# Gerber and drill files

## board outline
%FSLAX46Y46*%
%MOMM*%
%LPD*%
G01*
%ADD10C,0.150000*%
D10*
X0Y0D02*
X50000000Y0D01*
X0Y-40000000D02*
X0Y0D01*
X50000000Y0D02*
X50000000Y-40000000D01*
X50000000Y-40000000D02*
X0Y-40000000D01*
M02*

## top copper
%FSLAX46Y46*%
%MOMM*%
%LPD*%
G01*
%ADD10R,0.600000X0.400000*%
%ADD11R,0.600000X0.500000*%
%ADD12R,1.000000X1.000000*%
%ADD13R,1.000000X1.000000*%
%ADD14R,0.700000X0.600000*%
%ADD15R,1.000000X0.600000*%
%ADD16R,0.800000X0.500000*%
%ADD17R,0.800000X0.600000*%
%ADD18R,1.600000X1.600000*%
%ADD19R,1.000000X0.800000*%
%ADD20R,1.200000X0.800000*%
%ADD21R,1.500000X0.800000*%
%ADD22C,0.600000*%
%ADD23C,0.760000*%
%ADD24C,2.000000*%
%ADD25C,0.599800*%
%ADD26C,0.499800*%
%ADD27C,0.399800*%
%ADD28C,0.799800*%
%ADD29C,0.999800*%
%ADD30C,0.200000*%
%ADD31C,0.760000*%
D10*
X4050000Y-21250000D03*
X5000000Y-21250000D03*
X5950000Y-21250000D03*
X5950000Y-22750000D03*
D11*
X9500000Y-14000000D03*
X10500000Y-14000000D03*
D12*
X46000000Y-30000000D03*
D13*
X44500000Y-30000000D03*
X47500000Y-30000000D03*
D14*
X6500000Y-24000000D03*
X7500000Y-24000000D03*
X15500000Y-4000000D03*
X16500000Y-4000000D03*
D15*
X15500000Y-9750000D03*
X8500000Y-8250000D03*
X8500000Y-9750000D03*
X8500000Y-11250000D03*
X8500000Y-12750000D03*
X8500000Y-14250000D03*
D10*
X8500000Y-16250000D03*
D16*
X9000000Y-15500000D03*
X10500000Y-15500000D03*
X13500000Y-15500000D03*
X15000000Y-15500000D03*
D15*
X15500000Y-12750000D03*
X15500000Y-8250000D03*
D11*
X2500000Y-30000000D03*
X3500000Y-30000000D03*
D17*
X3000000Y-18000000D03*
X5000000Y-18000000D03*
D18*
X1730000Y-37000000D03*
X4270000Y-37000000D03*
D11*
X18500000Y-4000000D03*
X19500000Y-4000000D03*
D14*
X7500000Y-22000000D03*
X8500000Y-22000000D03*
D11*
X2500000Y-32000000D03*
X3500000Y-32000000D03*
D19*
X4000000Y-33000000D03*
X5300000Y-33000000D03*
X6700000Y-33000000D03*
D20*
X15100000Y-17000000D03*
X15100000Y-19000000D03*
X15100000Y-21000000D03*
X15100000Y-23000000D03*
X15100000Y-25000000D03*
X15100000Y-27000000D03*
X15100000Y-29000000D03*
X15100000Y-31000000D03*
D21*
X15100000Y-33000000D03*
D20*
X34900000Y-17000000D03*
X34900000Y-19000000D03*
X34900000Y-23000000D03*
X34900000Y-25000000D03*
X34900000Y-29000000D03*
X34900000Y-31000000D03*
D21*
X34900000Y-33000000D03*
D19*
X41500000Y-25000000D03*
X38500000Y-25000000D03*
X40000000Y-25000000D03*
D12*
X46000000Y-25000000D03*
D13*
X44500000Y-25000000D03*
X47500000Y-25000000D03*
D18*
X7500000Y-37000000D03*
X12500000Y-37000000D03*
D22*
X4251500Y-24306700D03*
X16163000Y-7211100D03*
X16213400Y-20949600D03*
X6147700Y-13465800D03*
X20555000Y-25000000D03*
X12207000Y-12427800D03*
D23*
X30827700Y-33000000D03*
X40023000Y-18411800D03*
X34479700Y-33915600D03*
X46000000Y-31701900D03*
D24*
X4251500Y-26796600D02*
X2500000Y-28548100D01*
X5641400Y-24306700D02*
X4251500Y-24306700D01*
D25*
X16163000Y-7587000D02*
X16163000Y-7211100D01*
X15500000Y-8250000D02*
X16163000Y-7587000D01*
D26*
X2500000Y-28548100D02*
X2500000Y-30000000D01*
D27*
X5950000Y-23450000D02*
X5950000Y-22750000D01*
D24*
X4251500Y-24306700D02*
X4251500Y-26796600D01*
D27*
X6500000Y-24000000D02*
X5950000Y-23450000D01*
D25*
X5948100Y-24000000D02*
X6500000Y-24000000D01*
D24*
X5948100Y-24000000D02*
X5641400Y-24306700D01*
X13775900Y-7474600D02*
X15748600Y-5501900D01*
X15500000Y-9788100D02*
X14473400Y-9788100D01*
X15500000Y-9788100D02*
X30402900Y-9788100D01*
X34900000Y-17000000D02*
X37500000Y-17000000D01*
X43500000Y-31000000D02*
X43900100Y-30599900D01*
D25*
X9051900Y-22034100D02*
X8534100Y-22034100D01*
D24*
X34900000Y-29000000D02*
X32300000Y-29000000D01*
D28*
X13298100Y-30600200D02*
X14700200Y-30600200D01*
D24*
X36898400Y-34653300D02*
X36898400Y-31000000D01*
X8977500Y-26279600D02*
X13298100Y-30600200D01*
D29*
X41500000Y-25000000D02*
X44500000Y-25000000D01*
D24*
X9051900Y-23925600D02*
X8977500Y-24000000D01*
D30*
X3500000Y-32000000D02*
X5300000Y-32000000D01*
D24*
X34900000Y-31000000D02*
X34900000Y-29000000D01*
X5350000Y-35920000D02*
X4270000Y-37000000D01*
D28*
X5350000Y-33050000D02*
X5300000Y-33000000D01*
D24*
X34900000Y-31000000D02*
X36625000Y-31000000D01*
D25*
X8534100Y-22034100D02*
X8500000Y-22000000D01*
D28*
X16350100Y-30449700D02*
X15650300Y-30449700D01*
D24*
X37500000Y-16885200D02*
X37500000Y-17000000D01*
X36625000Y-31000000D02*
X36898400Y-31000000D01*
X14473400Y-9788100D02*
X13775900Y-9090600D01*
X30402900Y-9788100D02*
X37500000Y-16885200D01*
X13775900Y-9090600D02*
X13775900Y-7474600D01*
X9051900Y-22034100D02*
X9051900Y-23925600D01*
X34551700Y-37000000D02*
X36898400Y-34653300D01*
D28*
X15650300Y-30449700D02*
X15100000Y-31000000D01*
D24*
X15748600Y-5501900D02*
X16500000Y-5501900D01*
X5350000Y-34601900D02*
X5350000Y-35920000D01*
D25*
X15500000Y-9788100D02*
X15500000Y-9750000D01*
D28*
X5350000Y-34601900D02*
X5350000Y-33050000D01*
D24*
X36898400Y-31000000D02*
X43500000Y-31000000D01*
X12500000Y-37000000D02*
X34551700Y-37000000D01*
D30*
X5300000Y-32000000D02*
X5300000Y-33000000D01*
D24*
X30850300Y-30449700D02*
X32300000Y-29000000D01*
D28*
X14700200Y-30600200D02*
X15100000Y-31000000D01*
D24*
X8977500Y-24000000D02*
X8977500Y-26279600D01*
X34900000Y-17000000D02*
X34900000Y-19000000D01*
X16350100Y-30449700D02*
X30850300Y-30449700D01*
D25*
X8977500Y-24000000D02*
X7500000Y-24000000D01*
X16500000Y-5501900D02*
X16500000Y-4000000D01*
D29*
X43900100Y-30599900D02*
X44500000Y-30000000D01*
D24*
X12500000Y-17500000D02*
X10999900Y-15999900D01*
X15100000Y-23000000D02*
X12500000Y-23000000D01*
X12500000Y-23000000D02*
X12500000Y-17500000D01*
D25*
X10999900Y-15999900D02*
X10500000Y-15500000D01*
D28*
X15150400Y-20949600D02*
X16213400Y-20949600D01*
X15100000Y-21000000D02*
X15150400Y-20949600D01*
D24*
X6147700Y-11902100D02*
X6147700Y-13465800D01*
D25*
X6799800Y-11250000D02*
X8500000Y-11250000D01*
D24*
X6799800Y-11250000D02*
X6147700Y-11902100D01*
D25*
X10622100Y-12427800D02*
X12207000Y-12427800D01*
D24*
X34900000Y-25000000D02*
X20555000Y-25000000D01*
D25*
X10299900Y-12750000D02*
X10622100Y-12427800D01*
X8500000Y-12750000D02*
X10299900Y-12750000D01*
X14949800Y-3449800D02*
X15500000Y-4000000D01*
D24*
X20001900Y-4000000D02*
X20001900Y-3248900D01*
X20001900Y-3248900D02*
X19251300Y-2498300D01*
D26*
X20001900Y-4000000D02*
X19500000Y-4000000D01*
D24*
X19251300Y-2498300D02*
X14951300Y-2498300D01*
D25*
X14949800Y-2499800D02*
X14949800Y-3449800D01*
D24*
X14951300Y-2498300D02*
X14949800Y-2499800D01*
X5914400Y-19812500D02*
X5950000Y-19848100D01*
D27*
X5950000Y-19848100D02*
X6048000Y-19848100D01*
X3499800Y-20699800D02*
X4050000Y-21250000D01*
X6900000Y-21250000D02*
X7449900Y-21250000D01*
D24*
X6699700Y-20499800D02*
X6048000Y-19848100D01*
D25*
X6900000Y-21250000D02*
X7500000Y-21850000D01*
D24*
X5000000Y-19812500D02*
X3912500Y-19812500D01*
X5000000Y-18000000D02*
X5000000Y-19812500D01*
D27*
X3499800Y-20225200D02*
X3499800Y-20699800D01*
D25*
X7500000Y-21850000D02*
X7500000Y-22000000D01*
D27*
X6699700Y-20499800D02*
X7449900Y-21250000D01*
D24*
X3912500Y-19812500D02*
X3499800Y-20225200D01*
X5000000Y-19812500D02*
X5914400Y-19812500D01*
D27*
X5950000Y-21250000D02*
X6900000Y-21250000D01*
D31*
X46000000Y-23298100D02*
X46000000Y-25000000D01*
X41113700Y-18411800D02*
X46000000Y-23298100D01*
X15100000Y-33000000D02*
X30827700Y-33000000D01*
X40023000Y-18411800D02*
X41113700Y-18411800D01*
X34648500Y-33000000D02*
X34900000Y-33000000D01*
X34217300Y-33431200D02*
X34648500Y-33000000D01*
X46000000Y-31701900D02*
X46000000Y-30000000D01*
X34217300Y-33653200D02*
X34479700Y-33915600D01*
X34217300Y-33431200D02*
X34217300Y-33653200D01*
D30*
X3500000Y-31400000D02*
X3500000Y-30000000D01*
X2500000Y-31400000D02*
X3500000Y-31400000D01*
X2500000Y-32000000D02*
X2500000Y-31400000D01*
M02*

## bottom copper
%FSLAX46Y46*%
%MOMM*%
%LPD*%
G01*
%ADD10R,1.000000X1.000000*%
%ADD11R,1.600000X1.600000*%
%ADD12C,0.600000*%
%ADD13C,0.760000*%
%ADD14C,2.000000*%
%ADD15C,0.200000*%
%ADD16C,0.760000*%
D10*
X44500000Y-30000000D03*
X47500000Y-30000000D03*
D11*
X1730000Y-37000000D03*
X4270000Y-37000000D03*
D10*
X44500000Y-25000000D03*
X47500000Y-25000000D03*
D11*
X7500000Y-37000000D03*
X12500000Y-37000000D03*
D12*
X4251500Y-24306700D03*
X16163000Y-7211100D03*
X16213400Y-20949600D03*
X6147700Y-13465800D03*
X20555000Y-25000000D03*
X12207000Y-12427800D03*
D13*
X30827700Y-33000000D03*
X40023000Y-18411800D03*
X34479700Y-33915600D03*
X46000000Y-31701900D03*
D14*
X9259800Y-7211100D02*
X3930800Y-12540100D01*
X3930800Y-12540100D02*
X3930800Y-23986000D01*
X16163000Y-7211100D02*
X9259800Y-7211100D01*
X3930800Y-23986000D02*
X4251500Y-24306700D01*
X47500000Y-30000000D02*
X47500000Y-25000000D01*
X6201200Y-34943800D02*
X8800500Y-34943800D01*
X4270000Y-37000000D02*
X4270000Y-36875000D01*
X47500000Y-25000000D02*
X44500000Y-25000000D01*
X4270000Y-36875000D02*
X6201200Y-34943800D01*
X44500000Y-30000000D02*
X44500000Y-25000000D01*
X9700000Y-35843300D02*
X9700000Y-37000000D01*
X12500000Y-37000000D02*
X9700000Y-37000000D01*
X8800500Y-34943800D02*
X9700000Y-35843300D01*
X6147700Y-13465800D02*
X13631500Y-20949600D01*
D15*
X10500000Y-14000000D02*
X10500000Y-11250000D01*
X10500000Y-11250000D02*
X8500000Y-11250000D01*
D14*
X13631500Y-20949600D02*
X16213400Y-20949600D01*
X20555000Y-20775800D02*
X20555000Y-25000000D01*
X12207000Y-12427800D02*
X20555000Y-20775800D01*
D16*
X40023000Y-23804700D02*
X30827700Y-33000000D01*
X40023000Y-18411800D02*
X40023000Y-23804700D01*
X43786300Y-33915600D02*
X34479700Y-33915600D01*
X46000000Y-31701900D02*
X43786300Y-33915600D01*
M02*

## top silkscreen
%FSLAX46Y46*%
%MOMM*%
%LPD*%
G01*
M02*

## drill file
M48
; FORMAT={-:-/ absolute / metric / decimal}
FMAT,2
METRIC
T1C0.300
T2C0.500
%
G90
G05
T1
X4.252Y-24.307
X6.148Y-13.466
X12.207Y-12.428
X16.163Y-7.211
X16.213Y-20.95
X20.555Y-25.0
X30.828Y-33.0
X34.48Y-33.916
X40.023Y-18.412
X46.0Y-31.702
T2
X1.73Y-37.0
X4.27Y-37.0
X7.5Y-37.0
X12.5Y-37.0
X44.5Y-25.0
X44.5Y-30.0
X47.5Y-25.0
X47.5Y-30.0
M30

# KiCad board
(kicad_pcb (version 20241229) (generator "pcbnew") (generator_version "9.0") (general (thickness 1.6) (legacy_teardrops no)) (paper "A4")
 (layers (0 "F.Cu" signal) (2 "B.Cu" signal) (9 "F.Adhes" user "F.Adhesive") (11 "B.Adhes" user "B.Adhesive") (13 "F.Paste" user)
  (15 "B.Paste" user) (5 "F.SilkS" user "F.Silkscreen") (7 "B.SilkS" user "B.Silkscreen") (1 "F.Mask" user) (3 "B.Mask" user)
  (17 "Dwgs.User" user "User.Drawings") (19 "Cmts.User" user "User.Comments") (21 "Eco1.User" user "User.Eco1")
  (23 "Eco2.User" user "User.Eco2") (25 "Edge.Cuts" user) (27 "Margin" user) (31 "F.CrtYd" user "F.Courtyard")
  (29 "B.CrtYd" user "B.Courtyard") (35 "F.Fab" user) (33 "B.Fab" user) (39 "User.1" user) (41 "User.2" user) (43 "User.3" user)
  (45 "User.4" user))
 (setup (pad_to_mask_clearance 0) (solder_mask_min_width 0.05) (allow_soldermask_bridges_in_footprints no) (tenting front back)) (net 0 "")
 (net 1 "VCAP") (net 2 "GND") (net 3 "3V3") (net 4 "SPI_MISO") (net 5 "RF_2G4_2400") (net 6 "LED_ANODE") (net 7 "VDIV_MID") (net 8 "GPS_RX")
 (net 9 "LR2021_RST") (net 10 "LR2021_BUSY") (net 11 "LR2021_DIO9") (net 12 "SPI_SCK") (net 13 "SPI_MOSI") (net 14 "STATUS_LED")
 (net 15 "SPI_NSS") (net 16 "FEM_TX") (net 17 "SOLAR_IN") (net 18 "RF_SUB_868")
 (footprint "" (layer "F.Cu") (at 5 22)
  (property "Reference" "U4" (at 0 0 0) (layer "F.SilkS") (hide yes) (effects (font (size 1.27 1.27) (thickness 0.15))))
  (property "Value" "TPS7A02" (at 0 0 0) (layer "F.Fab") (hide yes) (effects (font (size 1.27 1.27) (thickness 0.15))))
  (pad "1" smd rect (at -0.95 -0.75) (size 0.6 0.4) (layers "F.Cu" "F.Mask") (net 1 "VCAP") (thermal_bridge_angle 45))
  (pad "2" smd rect (at 0 -0.75) (size 0.6 0.4) (layers "F.Cu" "F.Mask") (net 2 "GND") (thermal_bridge_angle 45))
  (pad "3" smd rect (at 0.95 -0.75) (size 0.6 0.4) (layers "F.Cu" "F.Mask") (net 1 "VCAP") (thermal_bridge_angle 45))
  (pad "4" smd rect (at 0.95 0.75) (size 0.6 0.4) (layers "F.Cu" "F.Mask") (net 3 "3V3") (thermal_bridge_angle 45)))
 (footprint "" (layer "F.Cu") (at 10 14)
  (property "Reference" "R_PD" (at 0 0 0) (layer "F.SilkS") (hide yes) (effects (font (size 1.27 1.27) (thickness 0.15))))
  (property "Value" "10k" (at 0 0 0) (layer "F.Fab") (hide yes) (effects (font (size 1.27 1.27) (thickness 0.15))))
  (pad "1" smd rect (at -0.5 0) (size 0.6 0.5) (layers "F.Cu" "F.Mask") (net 2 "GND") (thermal_bridge_angle 45))
  (pad "2" smd rect (at 0.5 0) (size 0.6 0.5) (layers "F.Cu" "F.Mask") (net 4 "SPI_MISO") (thermal_bridge_angle 45)))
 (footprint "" (layer "F.Cu") (at 46 30)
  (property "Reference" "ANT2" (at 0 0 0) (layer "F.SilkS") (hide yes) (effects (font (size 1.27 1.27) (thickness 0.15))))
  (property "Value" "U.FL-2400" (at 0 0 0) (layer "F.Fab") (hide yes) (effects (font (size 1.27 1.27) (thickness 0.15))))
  (pad "1" smd rect (at 0 0) (size 1 1) (layers "F.Cu" "F.Mask") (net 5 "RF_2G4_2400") (thermal_bridge_angle 45))
  (pad "2" thru_hole rect (at -1.5 0) (size 1 1) (drill 0.5) (layers "*.Cu" "*.Mask") (remove_unused_layers no) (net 2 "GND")
   (thermal_bridge_angle 45))
  (pad "3" thru_hole rect (at 1.5 0) (size 1 1) (drill 0.5) (layers "*.Cu" "*.Mask") (remove_unused_layers no) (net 2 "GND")
   (thermal_bridge_angle 45)))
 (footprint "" (layer "F.Cu") (at 7 24)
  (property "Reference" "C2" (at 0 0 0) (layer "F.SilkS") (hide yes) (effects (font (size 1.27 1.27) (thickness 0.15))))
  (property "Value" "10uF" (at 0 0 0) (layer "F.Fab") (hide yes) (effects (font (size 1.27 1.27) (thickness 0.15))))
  (pad "1" smd rect (at -0.5 0) (size 0.7 0.6) (layers "F.Cu" "F.Mask") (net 3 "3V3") (thermal_bridge_angle 45))
  (pad "2" smd rect (at 0.5 0) (size 0.7 0.6) (layers "F.Cu" "F.Mask") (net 2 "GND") (thermal_bridge_angle 45)))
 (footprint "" (layer "F.Cu") (at 16 4)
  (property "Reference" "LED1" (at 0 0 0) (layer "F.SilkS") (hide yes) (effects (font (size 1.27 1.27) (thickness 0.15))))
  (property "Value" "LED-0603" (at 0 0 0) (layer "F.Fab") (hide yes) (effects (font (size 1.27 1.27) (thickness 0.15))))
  (pad "A" smd rect (at -0.5 0) (size 0.7 0.6) (layers "F.Cu" "F.Mask") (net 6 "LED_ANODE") (thermal_bridge_angle 45))
  (pad "K" smd rect (at 0.5 0) (size 0.7 0.6) (layers "F.Cu" "F.Mask") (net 2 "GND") (thermal_bridge_angle 45)))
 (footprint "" (layer "F.Cu") (at 12 12)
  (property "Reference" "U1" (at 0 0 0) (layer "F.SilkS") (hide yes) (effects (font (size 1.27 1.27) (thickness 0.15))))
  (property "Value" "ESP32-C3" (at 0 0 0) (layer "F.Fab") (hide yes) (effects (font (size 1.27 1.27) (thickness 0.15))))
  (pad "GND" smd rect (at 3.5 -2.25) (size 1 0.6) (layers "F.Cu" "F.Mask") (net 2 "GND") (thermal_bridge_angle 45))
  (pad "GPIO0" smd rect (at -3.5 -3.75) (size 1 0.6) (layers "F.Cu" "F.Mask") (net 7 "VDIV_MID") (thermal_bridge_angle 45))
  (pad "GPIO1" smd rect (at -3.5 -2.25) (size 1 0.6) (layers "F.Cu" "F.Mask") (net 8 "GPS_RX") (thermal_bridge_angle 45))
  (pad "GPIO2" smd rect (at -3.5 -0.75) (size 1 0.6) (layers "F.Cu" "F.Mask") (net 4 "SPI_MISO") (thermal_bridge_angle 45))
  (pad "GPIO3" smd rect (at -3.5 0.75) (size 1 0.6) (layers "F.Cu" "F.Mask") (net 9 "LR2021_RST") (thermal_bridge_angle 45))
  (pad "GPIO4" smd rect (at -3.5 2.25) (size 1 0.6) (layers "F.Cu" "F.Mask") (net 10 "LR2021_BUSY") (thermal_bridge_angle 45))
  (pad "GPIO5" smd rect (at -3.5 4.25) (size 0.6 0.4) (layers "F.Cu" "F.Mask") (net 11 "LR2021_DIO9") (thermal_bridge_angle 45))
  (pad "GPIO6" smd rect (at -3 3.5) (size 0.8 0.5) (layers "F.Cu" "F.Mask") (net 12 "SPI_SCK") (thermal_bridge_angle 45))
  (pad "GPIO7" smd rect (at -1.5 3.5) (size 0.8 0.5) (layers "F.Cu" "F.Mask") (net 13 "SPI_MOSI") (thermal_bridge_angle 45))
  (pad "GPIO9" smd rect (at 1.5 3.5) (size 0.8 0.5) (layers "F.Cu" "F.Mask") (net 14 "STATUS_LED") (thermal_bridge_angle 45))
  (pad "GPIO10" smd rect (at 3 3.5) (size 0.8 0.5) (layers "F.Cu" "F.Mask") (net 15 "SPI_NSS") (thermal_bridge_angle 45))
  (pad "GPIO19" smd rect (at 3.5 0.75) (size 1 0.6) (layers "F.Cu" "F.Mask") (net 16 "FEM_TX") (thermal_bridge_angle 45))
  (pad "VCC" smd rect (at 3.5 -3.75) (size 1 0.6) (layers "F.Cu" "F.Mask") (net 3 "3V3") (thermal_bridge_angle 45)))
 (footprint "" (layer "F.Cu") (at 3 30)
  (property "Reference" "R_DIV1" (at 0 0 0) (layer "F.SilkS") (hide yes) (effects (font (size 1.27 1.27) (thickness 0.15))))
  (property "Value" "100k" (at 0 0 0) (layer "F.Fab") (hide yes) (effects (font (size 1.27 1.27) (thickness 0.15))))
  (pad "1" smd rect (at -0.5 0) (size 0.6 0.5) (layers "F.Cu" "F.Mask") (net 3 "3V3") (thermal_bridge_angle 45))
  (pad "2" smd rect (at 0.5 0) (size 0.6 0.5) (layers "F.Cu" "F.Mask") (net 7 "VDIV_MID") (thermal_bridge_angle 45)))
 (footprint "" (layer "F.Cu") (at 4 18)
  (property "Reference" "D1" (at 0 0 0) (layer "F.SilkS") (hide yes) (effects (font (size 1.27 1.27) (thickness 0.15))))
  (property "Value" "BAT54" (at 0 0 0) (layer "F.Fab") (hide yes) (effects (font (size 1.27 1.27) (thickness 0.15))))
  (pad "A" smd rect (at -1 0) (size 0.8 0.6) (layers "F.Cu" "F.Mask") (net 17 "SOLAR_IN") (thermal_bridge_angle 45))
  (pad "K" smd rect (at 1 0) (size 0.8 0.6) (layers "F.Cu" "F.Mask") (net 1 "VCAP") (thermal_bridge_angle 45)))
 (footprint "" (layer "F.Cu") (at 3 37)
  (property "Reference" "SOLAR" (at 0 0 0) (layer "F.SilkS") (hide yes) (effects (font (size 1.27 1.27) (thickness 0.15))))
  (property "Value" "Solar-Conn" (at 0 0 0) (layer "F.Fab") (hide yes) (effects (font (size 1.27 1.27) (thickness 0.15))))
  (pad "1" thru_hole rect (at -1.27 0) (size 1.6 1.6) (drill 0.5) (layers "*.Cu" "*.Mask") (remove_unused_layers no) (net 17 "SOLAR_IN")
   (thermal_bridge_angle 45))
  (pad "2" thru_hole rect (at 1.27 0) (size 1.6 1.6) (drill 0.5) (layers "*.Cu" "*.Mask") (remove_unused_layers no) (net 2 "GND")
   (thermal_bridge_angle 45)))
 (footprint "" (layer "F.Cu") (at 19 4)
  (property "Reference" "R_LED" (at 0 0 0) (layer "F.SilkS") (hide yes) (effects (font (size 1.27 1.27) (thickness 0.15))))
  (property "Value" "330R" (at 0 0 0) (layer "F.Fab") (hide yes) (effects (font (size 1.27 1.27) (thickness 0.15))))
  (pad "1" smd rect (at -0.5 0) (size 0.6 0.5) (layers "F.Cu" "F.Mask") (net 14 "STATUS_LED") (thermal_bridge_angle 45))
  (pad "2" smd rect (at 0.5 0) (size 0.6 0.5) (layers "F.Cu" "F.Mask") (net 6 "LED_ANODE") (thermal_bridge_angle 45)))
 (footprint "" (layer "F.Cu") (at 8 22)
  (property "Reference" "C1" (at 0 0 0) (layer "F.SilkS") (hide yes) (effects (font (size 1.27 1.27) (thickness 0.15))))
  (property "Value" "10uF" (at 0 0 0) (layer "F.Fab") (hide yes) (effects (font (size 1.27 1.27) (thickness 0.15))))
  (pad "1" smd rect (at -0.5 0) (size 0.7 0.6) (layers "F.Cu" "F.Mask") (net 1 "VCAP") (thermal_bridge_angle 45))
  (pad "2" smd rect (at 0.5 0) (size 0.7 0.6) (layers "F.Cu" "F.Mask") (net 2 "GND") (thermal_bridge_angle 45)))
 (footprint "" (layer "F.Cu") (at 3 32)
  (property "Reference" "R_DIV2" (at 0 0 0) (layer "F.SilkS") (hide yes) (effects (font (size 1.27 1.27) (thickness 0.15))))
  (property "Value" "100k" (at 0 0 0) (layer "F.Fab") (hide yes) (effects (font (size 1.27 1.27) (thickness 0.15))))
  (pad "1" smd rect (at -0.5 0) (size 0.6 0.5) (layers "F.Cu" "F.Mask") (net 7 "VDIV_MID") (thermal_bridge_angle 45))
  (pad "2" smd rect (at 0.5 0) (size 0.6 0.5) (layers "F.Cu" "F.Mask") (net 2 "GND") (thermal_bridge_angle 45)))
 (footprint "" (layer "F.Cu") (at 6 33)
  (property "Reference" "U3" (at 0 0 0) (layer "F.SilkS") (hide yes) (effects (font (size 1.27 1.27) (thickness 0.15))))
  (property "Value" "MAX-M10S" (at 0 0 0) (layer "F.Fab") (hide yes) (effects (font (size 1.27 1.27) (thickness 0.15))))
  (pad "1" smd rect (at -2 0) (size 1 0.8) (layers "F.Cu" "F.Mask") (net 3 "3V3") (thermal_bridge_angle 45))
  (pad "2" smd rect (at -0.7 0) (size 1 0.8) (layers "F.Cu" "F.Mask") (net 2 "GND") (thermal_bridge_angle 45))
  (pad "3" smd rect (at 0.7 0) (size 1 0.8) (layers "F.Cu" "F.Mask") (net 8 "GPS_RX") (thermal_bridge_angle 45)))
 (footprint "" (layer "F.Cu") (at 25 25)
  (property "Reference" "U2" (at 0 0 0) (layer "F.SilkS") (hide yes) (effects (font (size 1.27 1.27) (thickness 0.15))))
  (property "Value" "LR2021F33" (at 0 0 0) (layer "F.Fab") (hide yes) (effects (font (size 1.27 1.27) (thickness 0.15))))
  (pad "1" smd rect (at -9.9 -8) (size 1.2 0.8) (layers "F.Cu" "F.Mask") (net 3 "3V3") (thermal_bridge_angle 45))
  (pad "2" smd rect (at -9.9 -6) (size 1.2 0.8) (layers "F.Cu" "F.Mask") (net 2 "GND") (thermal_bridge_angle 45))
  (pad "3" smd rect (at -9.9 -4) (size 1.2 0.8) (layers "F.Cu" "F.Mask") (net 4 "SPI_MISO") (thermal_bridge_angle 45))
  (pad "4" smd rect (at -9.9 -2) (size 1.2 0.8) (layers "F.Cu" "F.Mask") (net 13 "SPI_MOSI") (thermal_bridge_angle 45))
  (pad "5" smd rect (at -9.9 0) (size 1.2 0.8) (layers "F.Cu" "F.Mask") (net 12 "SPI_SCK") (thermal_bridge_angle 45))
  (pad "6" smd rect (at -9.9 2) (size 1.2 0.8) (layers "F.Cu" "F.Mask") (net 15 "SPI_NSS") (thermal_bridge_angle 45))
  (pad "7" smd rect (at -9.9 4) (size 1.2 0.8) (layers "F.Cu" "F.Mask") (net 10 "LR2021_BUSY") (thermal_bridge_angle 45))
  (pad "8" smd rect (at -9.9 6) (size 1.2 0.8) (layers "F.Cu" "F.Mask") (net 2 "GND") (thermal_bridge_angle 45))
  (pad "9" smd rect (at -9.9 8) (size 1.5 0.8) (layers "F.Cu" "F.Mask") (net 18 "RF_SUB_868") (thermal_bridge_angle 45))
  (pad "10" smd rect (at 9.9 -8) (size 1.2 0.8) (layers "F.Cu" "F.Mask") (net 2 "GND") (thermal_bridge_angle 45))
  (pad "11" smd rect (at 9.9 -6) (size 1.2 0.8) (layers "F.Cu" "F.Mask") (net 2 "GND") (thermal_bridge_angle 45))
  (pad "13" smd rect (at 9.9 -2) (size 1.2 0.8) (layers "F.Cu" "F.Mask") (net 11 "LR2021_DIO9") (thermal_bridge_angle 45))
  (pad "14" smd rect (at 9.9 0) (size 1.2 0.8) (layers "F.Cu" "F.Mask") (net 9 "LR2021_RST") (thermal_bridge_angle 45))
  (pad "16" smd rect (at 9.9 4) (size 1.2 0.8) (layers "F.Cu" "F.Mask") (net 2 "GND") (thermal_bridge_angle 45))
  (pad "17" smd rect (at 9.9 6) (size 1.2 0.8) (layers "F.Cu" "F.Mask") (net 2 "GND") (thermal_bridge_angle 45))
  (pad "18" smd rect (at 9.9 8) (size 1.5 0.8) (layers "F.Cu" "F.Mask") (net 5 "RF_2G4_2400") (thermal_bridge_angle 45)))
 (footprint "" (layer "F.Cu") (at 40 25)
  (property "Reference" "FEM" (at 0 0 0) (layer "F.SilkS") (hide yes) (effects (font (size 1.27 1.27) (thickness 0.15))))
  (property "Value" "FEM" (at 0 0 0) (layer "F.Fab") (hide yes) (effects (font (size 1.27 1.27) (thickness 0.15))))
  (pad "GND" smd rect (at 1.5 0) (size 1 0.8) (layers "F.Cu" "F.Mask") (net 2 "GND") (thermal_bridge_angle 45))
  (pad "TX" smd rect (at -1.5 0) (size 1 0.8) (layers "F.Cu" "F.Mask") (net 16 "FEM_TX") (thermal_bridge_angle 45))
  (pad "VCC" smd rect (at 0 0) (size 1 0.8) (layers "F.Cu" "F.Mask") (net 3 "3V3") (thermal_bridge_angle 45)))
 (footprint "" (layer "F.Cu") (at 46 25)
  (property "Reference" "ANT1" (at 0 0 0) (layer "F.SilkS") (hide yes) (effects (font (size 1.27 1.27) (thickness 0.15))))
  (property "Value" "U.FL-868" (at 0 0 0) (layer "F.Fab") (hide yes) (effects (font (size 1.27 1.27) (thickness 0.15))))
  (pad "1" smd rect (at 0 0) (size 1 1) (layers "F.Cu" "F.Mask") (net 18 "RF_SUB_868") (thermal_bridge_angle 45))
  (pad "2" thru_hole rect (at -1.5 0) (size 1 1) (drill 0.5) (layers "*.Cu" "*.Mask") (remove_unused_layers no) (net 2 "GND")
   (thermal_bridge_angle 45))
  (pad "3" thru_hole rect (at 1.5 0) (size 1 1) (drill 0.5) (layers "*.Cu" "*.Mask") (remove_unused_layers no) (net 2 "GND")
   (thermal_bridge_angle 45)))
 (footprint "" (layer "F.Cu") (at 10 37)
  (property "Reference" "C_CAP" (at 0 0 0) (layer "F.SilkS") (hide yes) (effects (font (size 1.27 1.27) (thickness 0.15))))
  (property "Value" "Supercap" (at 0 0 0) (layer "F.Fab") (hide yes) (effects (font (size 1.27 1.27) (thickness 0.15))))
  (pad "1" thru_hole rect (at -2.5 0) (size 1.6 1.6) (drill 0.5) (layers "*.Cu" "*.Mask") (remove_unused_layers no) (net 1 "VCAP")
   (thermal_bridge_angle 45))
  (pad "2" thru_hole rect (at 2.5 0) (size 1.6 1.6) (drill 0.5) (layers "*.Cu" "*.Mask") (remove_unused_layers no) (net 2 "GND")
   (thermal_bridge_angle 45)))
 (gr_line (start 0 0) (end 50 0) (stroke (width 0.15) (type default)) (layer "Edge.Cuts"))
 (gr_line (start 0 40) (end 0 0) (stroke (width 0.15) (type default)) (layer "Edge.Cuts"))
 (gr_line (start 50 0) (end 50 40) (stroke (width 0.15) (type default)) (layer "Edge.Cuts"))
 (gr_line (start 50 40) (end 0 40) (stroke (width 0.15) (type default)) (layer "Edge.Cuts"))
 (segment (start 4.2515 26.7966) (end 2.5 28.5481) (width 2) (layer "F.Cu") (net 3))
 (segment (start 5.6414 24.3067) (end 4.2515 24.3067) (width 2) (layer "F.Cu") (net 3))
 (segment (start 16.163 7.587) (end 16.163 7.2111) (width 0.5998) (layer "F.Cu") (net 3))
 (segment (start 15.5 8.25) (end 16.163 7.587) (width 0.5998) (layer "F.Cu") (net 3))
 (segment (start 2.5 28.5481) (end 2.5 30) (width 0.4998) (layer "F.Cu") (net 3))
 (segment (start 5.95 23.45) (end 5.95 22.75) (width 0.3998) (layer "F.Cu") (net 3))
 (segment (start 4.2515 24.3067) (end 4.2515 26.7966) (width 2) (layer "F.Cu") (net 3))
 (segment (start 6.5 24) (end 5.95 23.45) (width 0.3998) (layer "F.Cu") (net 3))
 (segment (start 5.9481 24) (end 6.5 24) (width 0.5998) (layer "F.Cu") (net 3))
 (segment (start 5.9481 24) (end 5.6414 24.3067) (width 2) (layer "F.Cu") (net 3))
 (via (at 4.2515 24.3067) (size 0.6) (drill 0.3) (layers "F.Cu" "B.Cu") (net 3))
 (via (at 16.163 7.2111) (size 0.6) (drill 0.3) (layers "F.Cu" "B.Cu") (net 3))
 (segment (start 9.2598 7.2111) (end 3.9308 12.5401) (width 2) (layer "B.Cu") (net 3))
 (segment (start 3.9308 12.5401) (end 3.9308 23.986) (width 2) (layer "B.Cu") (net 3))
 (segment (start 16.163 7.2111) (end 9.2598 7.2111) (width 2) (layer "B.Cu") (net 3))
 (segment (start 3.9308 23.986) (end 4.2515 24.3067) (width 2) (layer "B.Cu") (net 3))
 (segment (start 13.7759 7.4746) (end 15.7486 5.5019) (width 2) (layer "F.Cu") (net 2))
 (segment (start 15.5 9.7881) (end 14.4734 9.7881) (width 2) (layer "F.Cu") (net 2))
 (segment (start 15.5 9.7881) (end 30.4029 9.7881) (width 2) (layer "F.Cu") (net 2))
 (segment (start 34.9 17) (end 37.5 17) (width 2) (layer "F.Cu") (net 2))
 (segment (start 43.5 31) (end 43.9001 30.5999) (width 2) (layer "F.Cu") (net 2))
 (segment (start 9.0519 22.0341) (end 8.5341 22.0341) (width 0.5998) (layer "F.Cu") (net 2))
 (segment (start 34.9 29) (end 32.3 29) (width 2) (layer "F.Cu") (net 2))
 (segment (start 13.2981 30.6002) (end 14.7002 30.6002) (width 0.7998) (layer "F.Cu") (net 2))
 (segment (start 36.8984 34.6533) (end 36.8984 31) (width 2) (layer "F.Cu") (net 2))
 (segment (start 8.9775 26.2796) (end 13.2981 30.6002) (width 2) (layer "F.Cu") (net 2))
 (segment (start 41.5 25) (end 44.5 25) (width 0.9998) (layer "F.Cu") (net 2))
 (segment (start 9.0519 23.9256) (end 8.9775 24) (width 2) (layer "F.Cu") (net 2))
 (segment (start 3.5 32) (end 5.3 32) (width 0.2) (layer "F.Cu") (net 2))
 (segment (start 34.9 31) (end 34.9 29) (width 2) (layer "F.Cu") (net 2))
 (segment (start 5.35 35.92) (end 4.27 37) (width 2) (layer "F.Cu") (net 2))
 (segment (start 5.35 33.05) (end 5.3 33) (width 0.7998) (layer "F.Cu") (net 2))
 (segment (start 34.9 31) (end 36.625 31) (width 2) (layer "F.Cu") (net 2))
 (segment (start 8.5341 22.0341) (end 8.5 22) (width 0.5998) (layer "F.Cu") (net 2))
 (segment (start 16.3501 30.4497) (end 15.6503 30.4497) (width 0.7998) (layer "F.Cu") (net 2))
 (segment (start 37.5 16.8852) (end 37.5 17) (width 2) (layer "F.Cu") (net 2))
 (segment (start 36.625 31) (end 36.8984 31) (width 2) (layer "F.Cu") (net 2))
 (segment (start 14.4734 9.7881) (end 13.7759 9.0906) (width 2) (layer "F.Cu") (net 2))
 (segment (start 30.4029 9.7881) (end 37.5 16.8852) (width 2) (layer "F.Cu") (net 2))
 (segment (start 13.7759 9.0906) (end 13.7759 7.4746) (width 2) (layer "F.Cu") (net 2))
 (segment (start 9.0519 22.0341) (end 9.0519 23.9256) (width 2) (layer "F.Cu") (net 2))
 (segment (start 34.5517 37) (end 36.8984 34.6533) (width 2) (layer "F.Cu") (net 2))
 (segment (start 15.6503 30.4497) (end 15.1 31) (width 0.7998) (layer "F.Cu") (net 2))
 (segment (start 15.7486 5.5019) (end 16.5 5.5019) (width 2) (layer "F.Cu") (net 2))
 (segment (start 5.35 34.6019) (end 5.35 35.92) (width 2) (layer "F.Cu") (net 2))
 (segment (start 15.5 9.7881) (end 15.5 9.75) (width 0.5998) (layer "F.Cu") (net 2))
 (segment (start 5.35 34.6019) (end 5.35 33.05) (width 0.7998) (layer "F.Cu") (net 2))
 (segment (start 36.8984 31) (end 43.5 31) (width 2) (layer "F.Cu") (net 2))
 (segment (start 12.5 37) (end 34.5517 37) (width 2) (layer "F.Cu") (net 2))
 (segment (start 5.3 32) (end 5.3 33) (width 0.2) (layer "F.Cu") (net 2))
 (segment (start 30.8503 30.4497) (end 32.3 29) (width 2) (layer "F.Cu") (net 2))
 (segment (start 14.7002 30.6002) (end 15.1 31) (width 0.7998) (layer "F.Cu") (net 2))
 (segment (start 8.9775 24) (end 8.9775 26.2796) (width 2) (layer "F.Cu") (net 2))
 (segment (start 34.9 17) (end 34.9 19) (width 2) (layer "F.Cu") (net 2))
 (segment (start 16.3501 30.4497) (end 30.8503 30.4497) (width 2) (layer "F.Cu") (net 2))
 (segment (start 8.9775 24) (end 7.5 24) (width 0.5998) (layer "F.Cu") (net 2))
 (segment (start 16.5 5.5019) (end 16.5 4) (width 0.5998) (layer "F.Cu") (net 2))
 (segment (start 43.9001 30.5999) (end 44.5 30) (width 0.9998) (layer "F.Cu") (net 2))
 (segment (start 47.5 30) (end 47.5 25) (width 2) (layer "B.Cu") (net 2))
 (segment (start 6.2012 34.9438) (end 8.8005 34.9438) (width 2) (layer "B.Cu") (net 2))
 (segment (start 4.27 37) (end 4.27 36.875) (width 2) (layer "B.Cu") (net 2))
 (segment (start 47.5 25) (end 44.5 25) (width 2) (layer "B.Cu") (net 2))
 (segment (start 4.27 36.875) (end 6.2012 34.9438) (width 2) (layer "B.Cu") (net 2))
 (segment (start 44.5 30) (end 44.5 25) (width 2) (layer "B.Cu") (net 2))
 (segment (start 9.7 35.8433) (end 9.7 37) (width 2) (layer "B.Cu") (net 2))
 (segment (start 12.5 37) (end 9.7 37) (width 2) (layer "B.Cu") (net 2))
 (segment (start 8.8005 34.9438) (end 9.7 35.8433) (width 2) (layer "B.Cu") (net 2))
 (segment (start 12.5 17.5) (end 10.9999 15.9999) (width 2) (layer "F.Cu") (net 13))
 (segment (start 15.1 23) (end 12.5 23) (width 2) (layer "F.Cu") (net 13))
 (segment (start 12.5 23) (end 12.5 17.5) (width 2) (layer "F.Cu") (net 13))
 (segment (start 10.9999 15.9999) (end 10.5 15.5) (width 0.5998) (layer "F.Cu") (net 13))
 (segment (start 15.1504 20.9496) (end 16.2134 20.9496) (width 0.7998) (layer "F.Cu") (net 4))
 (segment (start 15.1 21) (end 15.1504 20.9496) (width 0.7998) (layer "F.Cu") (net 4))
 (segment (start 6.1477 11.9021) (end 6.1477 13.4658) (width 2) (layer "F.Cu") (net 4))
 (segment (start 6.7998 11.25) (end 8.5 11.25) (width 0.5998) (layer "F.Cu") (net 4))
 (segment (start 6.7998 11.25) (end 6.1477 11.9021) (width 2) (layer "F.Cu") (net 4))
 (via (at 16.2134 20.9496) (size 0.6) (drill 0.3) (layers "F.Cu" "B.Cu") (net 4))
 (via (at 6.1477 13.4658) (size 0.6) (drill 0.3) (layers "F.Cu" "B.Cu") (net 4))
 (segment (start 6.1477 13.4658) (end 13.6315 20.9496) (width 2) (layer "B.Cu") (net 4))
 (segment (start 10.5 14) (end 10.5 11.25) (width 0.2) (layer "B.Cu") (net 4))
 (segment (start 10.5 11.25) (end 8.5 11.25) (width 0.2) (layer "B.Cu") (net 4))
 (segment (start 13.6315 20.9496) (end 16.2134 20.9496) (width 2) (layer "B.Cu") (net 4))
 (segment (start 10.6221 12.4278) (end 12.207 12.4278) (width 0.5998) (layer "F.Cu") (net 9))
 (segment (start 34.9 25) (end 20.555 25) (width 2) (layer "F.Cu") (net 9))
 (segment (start 10.2999 12.75) (end 10.6221 12.4278) (width 0.5998) (layer "F.Cu") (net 9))
 (segment (start 8.5 12.75) (end 10.2999 12.75) (width 0.5998) (layer "F.Cu") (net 9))
 (via (at 20.555 25) (size 0.6) (drill 0.3) (layers "F.Cu" "B.Cu") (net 9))
 (via (at 12.207 12.4278) (size 0.6) (drill 0.3) (layers "F.Cu" "B.Cu") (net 9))
 (segment (start 20.555 20.7758) (end 20.555 25) (width 2) (layer "B.Cu") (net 9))
 (segment (start 12.207 12.4278) (end 20.555 20.7758) (width 2) (layer "B.Cu") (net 9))
 (segment (start 14.9498 3.4498) (end 15.5 4) (width 0.5998) (layer "F.Cu") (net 6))
 (segment (start 20.0019 4) (end 20.0019 3.2489) (width 2) (layer "F.Cu") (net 6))
 (segment (start 20.0019 3.2489) (end 19.2513 2.4983) (width 2) (layer "F.Cu") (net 6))
 (segment (start 20.0019 4) (end 19.5 4) (width 0.4998) (layer "F.Cu") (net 6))
 (segment (start 19.2513 2.4983) (end 14.9513 2.4983) (width 2) (layer "F.Cu") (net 6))
 (segment (start 14.9498 2.4998) (end 14.9498 3.4498) (width 0.5998) (layer "F.Cu") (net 6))
 (segment (start 14.9513 2.4983) (end 14.9498 2.4998) (width 2) (layer "F.Cu") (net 6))
 (segment (start 5.9144 19.8125) (end 5.95 19.8481) (width 2) (layer "F.Cu") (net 1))
 (segment (start 5.95 19.8481) (end 6.048 19.8481) (width 0.3998) (layer "F.Cu") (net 1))
 (segment (start 3.4998 20.6998) (end 4.05 21.25) (width 0.3998) (layer "F.Cu") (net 1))
 (segment (start 6.9 21.25) (end 7.4499 21.25) (width 0.3998) (layer "F.Cu") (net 1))
 (segment (start 6.6997 20.4998) (end 6.048 19.8481) (width 2) (layer "F.Cu") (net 1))
 (segment (start 6.9 21.25) (end 7.5 21.85) (width 0.5998) (layer "F.Cu") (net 1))
 (segment (start 5 19.8125) (end 3.9125 19.8125) (width 2) (layer "F.Cu") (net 1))
 (segment (start 5 18) (end 5 19.8125) (width 2) (layer "F.Cu") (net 1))
 (segment (start 3.4998 20.2252) (end 3.4998 20.6998) (width 0.3998) (layer "F.Cu") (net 1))
 (segment (start 7.5 21.85) (end 7.5 22) (width 0.5998) (layer "F.Cu") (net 1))
 (segment (start 6.6997 20.4998) (end 7.4499 21.25) (width 0.3998) (layer "F.Cu") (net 1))
 (segment (start 3.9125 19.8125) (end 3.4998 20.2252) (width 2) (layer "F.Cu") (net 1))
 (segment (start 5 19.8125) (end 5.9144 19.8125) (width 2) (layer "F.Cu") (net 1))
 (segment (start 5.95 21.25) (end 6.9 21.25) (width 0.3998) (layer "F.Cu") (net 1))
 (segment (start 46 23.2981) (end 46 25) (width 0.76) (layer "F.Cu") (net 18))
 (segment (start 41.1137 18.4118) (end 46 23.2981) (width 0.76) (layer "F.Cu") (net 18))
 (segment (start 15.1 33) (end 30.8277 33) (width 0.76) (layer "F.Cu") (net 18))
 (segment (start 40.023 18.4118) (end 41.1137 18.4118) (width 0.76) (layer "F.Cu") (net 18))
 (via (at 30.8277 33) (size 0.76) (drill 0.3) (layers "F.Cu" "B.Cu") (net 18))
 (via (at 40.023 18.4118) (size 0.76) (drill 0.3) (layers "F.Cu" "B.Cu") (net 18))
 (segment (start 40.023 23.8047) (end 30.8277 33) (width 0.76) (layer "B.Cu") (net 18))
 (segment (start 40.023 18.4118) (end 40.023 23.8047) (width 0.76) (layer "B.Cu") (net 18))
 (segment (start 34.6485 33) (end 34.9 33) (width 0.76) (layer "F.Cu") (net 5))
 (segment (start 34.2173 33.4312) (end 34.6485 33) (width 0.76) (layer "F.Cu") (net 5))
 (segment (start 46 31.7019) (end 46 30) (width 0.76) (layer "F.Cu") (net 5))
 (segment (start 34.2173 33.6532) (end 34.4797 33.9156) (width 0.76) (layer "F.Cu") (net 5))
 (segment (start 34.2173 33.4312) (end 34.2173 33.6532) (width 0.76) (layer "F.Cu") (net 5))
 (via (at 34.4797 33.9156) (size 0.76) (drill 0.3) (layers "F.Cu" "B.Cu") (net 5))
 (via (at 46 31.7019) (size 0.76) (drill 0.3) (layers "F.Cu" "B.Cu") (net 5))
 (segment (start 43.7863 33.9156) (end 34.4797 33.9156) (width 0.76) (layer "B.Cu") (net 5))
 (segment (start 46 31.7019) (end 43.7863 33.9156) (width 0.76) (layer "B.Cu") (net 5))
 (segment (start 3.5 31.4) (end 3.5 30) (width 0.2) (layer "F.Cu") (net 7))
 (segment (start 2.5 31.4) (end 3.5 31.4) (width 0.2) (layer "F.Cu") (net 7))
 (segment (start 2.5 32) (end 2.5 31.4) (width 0.2) (layer "F.Cu") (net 7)))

